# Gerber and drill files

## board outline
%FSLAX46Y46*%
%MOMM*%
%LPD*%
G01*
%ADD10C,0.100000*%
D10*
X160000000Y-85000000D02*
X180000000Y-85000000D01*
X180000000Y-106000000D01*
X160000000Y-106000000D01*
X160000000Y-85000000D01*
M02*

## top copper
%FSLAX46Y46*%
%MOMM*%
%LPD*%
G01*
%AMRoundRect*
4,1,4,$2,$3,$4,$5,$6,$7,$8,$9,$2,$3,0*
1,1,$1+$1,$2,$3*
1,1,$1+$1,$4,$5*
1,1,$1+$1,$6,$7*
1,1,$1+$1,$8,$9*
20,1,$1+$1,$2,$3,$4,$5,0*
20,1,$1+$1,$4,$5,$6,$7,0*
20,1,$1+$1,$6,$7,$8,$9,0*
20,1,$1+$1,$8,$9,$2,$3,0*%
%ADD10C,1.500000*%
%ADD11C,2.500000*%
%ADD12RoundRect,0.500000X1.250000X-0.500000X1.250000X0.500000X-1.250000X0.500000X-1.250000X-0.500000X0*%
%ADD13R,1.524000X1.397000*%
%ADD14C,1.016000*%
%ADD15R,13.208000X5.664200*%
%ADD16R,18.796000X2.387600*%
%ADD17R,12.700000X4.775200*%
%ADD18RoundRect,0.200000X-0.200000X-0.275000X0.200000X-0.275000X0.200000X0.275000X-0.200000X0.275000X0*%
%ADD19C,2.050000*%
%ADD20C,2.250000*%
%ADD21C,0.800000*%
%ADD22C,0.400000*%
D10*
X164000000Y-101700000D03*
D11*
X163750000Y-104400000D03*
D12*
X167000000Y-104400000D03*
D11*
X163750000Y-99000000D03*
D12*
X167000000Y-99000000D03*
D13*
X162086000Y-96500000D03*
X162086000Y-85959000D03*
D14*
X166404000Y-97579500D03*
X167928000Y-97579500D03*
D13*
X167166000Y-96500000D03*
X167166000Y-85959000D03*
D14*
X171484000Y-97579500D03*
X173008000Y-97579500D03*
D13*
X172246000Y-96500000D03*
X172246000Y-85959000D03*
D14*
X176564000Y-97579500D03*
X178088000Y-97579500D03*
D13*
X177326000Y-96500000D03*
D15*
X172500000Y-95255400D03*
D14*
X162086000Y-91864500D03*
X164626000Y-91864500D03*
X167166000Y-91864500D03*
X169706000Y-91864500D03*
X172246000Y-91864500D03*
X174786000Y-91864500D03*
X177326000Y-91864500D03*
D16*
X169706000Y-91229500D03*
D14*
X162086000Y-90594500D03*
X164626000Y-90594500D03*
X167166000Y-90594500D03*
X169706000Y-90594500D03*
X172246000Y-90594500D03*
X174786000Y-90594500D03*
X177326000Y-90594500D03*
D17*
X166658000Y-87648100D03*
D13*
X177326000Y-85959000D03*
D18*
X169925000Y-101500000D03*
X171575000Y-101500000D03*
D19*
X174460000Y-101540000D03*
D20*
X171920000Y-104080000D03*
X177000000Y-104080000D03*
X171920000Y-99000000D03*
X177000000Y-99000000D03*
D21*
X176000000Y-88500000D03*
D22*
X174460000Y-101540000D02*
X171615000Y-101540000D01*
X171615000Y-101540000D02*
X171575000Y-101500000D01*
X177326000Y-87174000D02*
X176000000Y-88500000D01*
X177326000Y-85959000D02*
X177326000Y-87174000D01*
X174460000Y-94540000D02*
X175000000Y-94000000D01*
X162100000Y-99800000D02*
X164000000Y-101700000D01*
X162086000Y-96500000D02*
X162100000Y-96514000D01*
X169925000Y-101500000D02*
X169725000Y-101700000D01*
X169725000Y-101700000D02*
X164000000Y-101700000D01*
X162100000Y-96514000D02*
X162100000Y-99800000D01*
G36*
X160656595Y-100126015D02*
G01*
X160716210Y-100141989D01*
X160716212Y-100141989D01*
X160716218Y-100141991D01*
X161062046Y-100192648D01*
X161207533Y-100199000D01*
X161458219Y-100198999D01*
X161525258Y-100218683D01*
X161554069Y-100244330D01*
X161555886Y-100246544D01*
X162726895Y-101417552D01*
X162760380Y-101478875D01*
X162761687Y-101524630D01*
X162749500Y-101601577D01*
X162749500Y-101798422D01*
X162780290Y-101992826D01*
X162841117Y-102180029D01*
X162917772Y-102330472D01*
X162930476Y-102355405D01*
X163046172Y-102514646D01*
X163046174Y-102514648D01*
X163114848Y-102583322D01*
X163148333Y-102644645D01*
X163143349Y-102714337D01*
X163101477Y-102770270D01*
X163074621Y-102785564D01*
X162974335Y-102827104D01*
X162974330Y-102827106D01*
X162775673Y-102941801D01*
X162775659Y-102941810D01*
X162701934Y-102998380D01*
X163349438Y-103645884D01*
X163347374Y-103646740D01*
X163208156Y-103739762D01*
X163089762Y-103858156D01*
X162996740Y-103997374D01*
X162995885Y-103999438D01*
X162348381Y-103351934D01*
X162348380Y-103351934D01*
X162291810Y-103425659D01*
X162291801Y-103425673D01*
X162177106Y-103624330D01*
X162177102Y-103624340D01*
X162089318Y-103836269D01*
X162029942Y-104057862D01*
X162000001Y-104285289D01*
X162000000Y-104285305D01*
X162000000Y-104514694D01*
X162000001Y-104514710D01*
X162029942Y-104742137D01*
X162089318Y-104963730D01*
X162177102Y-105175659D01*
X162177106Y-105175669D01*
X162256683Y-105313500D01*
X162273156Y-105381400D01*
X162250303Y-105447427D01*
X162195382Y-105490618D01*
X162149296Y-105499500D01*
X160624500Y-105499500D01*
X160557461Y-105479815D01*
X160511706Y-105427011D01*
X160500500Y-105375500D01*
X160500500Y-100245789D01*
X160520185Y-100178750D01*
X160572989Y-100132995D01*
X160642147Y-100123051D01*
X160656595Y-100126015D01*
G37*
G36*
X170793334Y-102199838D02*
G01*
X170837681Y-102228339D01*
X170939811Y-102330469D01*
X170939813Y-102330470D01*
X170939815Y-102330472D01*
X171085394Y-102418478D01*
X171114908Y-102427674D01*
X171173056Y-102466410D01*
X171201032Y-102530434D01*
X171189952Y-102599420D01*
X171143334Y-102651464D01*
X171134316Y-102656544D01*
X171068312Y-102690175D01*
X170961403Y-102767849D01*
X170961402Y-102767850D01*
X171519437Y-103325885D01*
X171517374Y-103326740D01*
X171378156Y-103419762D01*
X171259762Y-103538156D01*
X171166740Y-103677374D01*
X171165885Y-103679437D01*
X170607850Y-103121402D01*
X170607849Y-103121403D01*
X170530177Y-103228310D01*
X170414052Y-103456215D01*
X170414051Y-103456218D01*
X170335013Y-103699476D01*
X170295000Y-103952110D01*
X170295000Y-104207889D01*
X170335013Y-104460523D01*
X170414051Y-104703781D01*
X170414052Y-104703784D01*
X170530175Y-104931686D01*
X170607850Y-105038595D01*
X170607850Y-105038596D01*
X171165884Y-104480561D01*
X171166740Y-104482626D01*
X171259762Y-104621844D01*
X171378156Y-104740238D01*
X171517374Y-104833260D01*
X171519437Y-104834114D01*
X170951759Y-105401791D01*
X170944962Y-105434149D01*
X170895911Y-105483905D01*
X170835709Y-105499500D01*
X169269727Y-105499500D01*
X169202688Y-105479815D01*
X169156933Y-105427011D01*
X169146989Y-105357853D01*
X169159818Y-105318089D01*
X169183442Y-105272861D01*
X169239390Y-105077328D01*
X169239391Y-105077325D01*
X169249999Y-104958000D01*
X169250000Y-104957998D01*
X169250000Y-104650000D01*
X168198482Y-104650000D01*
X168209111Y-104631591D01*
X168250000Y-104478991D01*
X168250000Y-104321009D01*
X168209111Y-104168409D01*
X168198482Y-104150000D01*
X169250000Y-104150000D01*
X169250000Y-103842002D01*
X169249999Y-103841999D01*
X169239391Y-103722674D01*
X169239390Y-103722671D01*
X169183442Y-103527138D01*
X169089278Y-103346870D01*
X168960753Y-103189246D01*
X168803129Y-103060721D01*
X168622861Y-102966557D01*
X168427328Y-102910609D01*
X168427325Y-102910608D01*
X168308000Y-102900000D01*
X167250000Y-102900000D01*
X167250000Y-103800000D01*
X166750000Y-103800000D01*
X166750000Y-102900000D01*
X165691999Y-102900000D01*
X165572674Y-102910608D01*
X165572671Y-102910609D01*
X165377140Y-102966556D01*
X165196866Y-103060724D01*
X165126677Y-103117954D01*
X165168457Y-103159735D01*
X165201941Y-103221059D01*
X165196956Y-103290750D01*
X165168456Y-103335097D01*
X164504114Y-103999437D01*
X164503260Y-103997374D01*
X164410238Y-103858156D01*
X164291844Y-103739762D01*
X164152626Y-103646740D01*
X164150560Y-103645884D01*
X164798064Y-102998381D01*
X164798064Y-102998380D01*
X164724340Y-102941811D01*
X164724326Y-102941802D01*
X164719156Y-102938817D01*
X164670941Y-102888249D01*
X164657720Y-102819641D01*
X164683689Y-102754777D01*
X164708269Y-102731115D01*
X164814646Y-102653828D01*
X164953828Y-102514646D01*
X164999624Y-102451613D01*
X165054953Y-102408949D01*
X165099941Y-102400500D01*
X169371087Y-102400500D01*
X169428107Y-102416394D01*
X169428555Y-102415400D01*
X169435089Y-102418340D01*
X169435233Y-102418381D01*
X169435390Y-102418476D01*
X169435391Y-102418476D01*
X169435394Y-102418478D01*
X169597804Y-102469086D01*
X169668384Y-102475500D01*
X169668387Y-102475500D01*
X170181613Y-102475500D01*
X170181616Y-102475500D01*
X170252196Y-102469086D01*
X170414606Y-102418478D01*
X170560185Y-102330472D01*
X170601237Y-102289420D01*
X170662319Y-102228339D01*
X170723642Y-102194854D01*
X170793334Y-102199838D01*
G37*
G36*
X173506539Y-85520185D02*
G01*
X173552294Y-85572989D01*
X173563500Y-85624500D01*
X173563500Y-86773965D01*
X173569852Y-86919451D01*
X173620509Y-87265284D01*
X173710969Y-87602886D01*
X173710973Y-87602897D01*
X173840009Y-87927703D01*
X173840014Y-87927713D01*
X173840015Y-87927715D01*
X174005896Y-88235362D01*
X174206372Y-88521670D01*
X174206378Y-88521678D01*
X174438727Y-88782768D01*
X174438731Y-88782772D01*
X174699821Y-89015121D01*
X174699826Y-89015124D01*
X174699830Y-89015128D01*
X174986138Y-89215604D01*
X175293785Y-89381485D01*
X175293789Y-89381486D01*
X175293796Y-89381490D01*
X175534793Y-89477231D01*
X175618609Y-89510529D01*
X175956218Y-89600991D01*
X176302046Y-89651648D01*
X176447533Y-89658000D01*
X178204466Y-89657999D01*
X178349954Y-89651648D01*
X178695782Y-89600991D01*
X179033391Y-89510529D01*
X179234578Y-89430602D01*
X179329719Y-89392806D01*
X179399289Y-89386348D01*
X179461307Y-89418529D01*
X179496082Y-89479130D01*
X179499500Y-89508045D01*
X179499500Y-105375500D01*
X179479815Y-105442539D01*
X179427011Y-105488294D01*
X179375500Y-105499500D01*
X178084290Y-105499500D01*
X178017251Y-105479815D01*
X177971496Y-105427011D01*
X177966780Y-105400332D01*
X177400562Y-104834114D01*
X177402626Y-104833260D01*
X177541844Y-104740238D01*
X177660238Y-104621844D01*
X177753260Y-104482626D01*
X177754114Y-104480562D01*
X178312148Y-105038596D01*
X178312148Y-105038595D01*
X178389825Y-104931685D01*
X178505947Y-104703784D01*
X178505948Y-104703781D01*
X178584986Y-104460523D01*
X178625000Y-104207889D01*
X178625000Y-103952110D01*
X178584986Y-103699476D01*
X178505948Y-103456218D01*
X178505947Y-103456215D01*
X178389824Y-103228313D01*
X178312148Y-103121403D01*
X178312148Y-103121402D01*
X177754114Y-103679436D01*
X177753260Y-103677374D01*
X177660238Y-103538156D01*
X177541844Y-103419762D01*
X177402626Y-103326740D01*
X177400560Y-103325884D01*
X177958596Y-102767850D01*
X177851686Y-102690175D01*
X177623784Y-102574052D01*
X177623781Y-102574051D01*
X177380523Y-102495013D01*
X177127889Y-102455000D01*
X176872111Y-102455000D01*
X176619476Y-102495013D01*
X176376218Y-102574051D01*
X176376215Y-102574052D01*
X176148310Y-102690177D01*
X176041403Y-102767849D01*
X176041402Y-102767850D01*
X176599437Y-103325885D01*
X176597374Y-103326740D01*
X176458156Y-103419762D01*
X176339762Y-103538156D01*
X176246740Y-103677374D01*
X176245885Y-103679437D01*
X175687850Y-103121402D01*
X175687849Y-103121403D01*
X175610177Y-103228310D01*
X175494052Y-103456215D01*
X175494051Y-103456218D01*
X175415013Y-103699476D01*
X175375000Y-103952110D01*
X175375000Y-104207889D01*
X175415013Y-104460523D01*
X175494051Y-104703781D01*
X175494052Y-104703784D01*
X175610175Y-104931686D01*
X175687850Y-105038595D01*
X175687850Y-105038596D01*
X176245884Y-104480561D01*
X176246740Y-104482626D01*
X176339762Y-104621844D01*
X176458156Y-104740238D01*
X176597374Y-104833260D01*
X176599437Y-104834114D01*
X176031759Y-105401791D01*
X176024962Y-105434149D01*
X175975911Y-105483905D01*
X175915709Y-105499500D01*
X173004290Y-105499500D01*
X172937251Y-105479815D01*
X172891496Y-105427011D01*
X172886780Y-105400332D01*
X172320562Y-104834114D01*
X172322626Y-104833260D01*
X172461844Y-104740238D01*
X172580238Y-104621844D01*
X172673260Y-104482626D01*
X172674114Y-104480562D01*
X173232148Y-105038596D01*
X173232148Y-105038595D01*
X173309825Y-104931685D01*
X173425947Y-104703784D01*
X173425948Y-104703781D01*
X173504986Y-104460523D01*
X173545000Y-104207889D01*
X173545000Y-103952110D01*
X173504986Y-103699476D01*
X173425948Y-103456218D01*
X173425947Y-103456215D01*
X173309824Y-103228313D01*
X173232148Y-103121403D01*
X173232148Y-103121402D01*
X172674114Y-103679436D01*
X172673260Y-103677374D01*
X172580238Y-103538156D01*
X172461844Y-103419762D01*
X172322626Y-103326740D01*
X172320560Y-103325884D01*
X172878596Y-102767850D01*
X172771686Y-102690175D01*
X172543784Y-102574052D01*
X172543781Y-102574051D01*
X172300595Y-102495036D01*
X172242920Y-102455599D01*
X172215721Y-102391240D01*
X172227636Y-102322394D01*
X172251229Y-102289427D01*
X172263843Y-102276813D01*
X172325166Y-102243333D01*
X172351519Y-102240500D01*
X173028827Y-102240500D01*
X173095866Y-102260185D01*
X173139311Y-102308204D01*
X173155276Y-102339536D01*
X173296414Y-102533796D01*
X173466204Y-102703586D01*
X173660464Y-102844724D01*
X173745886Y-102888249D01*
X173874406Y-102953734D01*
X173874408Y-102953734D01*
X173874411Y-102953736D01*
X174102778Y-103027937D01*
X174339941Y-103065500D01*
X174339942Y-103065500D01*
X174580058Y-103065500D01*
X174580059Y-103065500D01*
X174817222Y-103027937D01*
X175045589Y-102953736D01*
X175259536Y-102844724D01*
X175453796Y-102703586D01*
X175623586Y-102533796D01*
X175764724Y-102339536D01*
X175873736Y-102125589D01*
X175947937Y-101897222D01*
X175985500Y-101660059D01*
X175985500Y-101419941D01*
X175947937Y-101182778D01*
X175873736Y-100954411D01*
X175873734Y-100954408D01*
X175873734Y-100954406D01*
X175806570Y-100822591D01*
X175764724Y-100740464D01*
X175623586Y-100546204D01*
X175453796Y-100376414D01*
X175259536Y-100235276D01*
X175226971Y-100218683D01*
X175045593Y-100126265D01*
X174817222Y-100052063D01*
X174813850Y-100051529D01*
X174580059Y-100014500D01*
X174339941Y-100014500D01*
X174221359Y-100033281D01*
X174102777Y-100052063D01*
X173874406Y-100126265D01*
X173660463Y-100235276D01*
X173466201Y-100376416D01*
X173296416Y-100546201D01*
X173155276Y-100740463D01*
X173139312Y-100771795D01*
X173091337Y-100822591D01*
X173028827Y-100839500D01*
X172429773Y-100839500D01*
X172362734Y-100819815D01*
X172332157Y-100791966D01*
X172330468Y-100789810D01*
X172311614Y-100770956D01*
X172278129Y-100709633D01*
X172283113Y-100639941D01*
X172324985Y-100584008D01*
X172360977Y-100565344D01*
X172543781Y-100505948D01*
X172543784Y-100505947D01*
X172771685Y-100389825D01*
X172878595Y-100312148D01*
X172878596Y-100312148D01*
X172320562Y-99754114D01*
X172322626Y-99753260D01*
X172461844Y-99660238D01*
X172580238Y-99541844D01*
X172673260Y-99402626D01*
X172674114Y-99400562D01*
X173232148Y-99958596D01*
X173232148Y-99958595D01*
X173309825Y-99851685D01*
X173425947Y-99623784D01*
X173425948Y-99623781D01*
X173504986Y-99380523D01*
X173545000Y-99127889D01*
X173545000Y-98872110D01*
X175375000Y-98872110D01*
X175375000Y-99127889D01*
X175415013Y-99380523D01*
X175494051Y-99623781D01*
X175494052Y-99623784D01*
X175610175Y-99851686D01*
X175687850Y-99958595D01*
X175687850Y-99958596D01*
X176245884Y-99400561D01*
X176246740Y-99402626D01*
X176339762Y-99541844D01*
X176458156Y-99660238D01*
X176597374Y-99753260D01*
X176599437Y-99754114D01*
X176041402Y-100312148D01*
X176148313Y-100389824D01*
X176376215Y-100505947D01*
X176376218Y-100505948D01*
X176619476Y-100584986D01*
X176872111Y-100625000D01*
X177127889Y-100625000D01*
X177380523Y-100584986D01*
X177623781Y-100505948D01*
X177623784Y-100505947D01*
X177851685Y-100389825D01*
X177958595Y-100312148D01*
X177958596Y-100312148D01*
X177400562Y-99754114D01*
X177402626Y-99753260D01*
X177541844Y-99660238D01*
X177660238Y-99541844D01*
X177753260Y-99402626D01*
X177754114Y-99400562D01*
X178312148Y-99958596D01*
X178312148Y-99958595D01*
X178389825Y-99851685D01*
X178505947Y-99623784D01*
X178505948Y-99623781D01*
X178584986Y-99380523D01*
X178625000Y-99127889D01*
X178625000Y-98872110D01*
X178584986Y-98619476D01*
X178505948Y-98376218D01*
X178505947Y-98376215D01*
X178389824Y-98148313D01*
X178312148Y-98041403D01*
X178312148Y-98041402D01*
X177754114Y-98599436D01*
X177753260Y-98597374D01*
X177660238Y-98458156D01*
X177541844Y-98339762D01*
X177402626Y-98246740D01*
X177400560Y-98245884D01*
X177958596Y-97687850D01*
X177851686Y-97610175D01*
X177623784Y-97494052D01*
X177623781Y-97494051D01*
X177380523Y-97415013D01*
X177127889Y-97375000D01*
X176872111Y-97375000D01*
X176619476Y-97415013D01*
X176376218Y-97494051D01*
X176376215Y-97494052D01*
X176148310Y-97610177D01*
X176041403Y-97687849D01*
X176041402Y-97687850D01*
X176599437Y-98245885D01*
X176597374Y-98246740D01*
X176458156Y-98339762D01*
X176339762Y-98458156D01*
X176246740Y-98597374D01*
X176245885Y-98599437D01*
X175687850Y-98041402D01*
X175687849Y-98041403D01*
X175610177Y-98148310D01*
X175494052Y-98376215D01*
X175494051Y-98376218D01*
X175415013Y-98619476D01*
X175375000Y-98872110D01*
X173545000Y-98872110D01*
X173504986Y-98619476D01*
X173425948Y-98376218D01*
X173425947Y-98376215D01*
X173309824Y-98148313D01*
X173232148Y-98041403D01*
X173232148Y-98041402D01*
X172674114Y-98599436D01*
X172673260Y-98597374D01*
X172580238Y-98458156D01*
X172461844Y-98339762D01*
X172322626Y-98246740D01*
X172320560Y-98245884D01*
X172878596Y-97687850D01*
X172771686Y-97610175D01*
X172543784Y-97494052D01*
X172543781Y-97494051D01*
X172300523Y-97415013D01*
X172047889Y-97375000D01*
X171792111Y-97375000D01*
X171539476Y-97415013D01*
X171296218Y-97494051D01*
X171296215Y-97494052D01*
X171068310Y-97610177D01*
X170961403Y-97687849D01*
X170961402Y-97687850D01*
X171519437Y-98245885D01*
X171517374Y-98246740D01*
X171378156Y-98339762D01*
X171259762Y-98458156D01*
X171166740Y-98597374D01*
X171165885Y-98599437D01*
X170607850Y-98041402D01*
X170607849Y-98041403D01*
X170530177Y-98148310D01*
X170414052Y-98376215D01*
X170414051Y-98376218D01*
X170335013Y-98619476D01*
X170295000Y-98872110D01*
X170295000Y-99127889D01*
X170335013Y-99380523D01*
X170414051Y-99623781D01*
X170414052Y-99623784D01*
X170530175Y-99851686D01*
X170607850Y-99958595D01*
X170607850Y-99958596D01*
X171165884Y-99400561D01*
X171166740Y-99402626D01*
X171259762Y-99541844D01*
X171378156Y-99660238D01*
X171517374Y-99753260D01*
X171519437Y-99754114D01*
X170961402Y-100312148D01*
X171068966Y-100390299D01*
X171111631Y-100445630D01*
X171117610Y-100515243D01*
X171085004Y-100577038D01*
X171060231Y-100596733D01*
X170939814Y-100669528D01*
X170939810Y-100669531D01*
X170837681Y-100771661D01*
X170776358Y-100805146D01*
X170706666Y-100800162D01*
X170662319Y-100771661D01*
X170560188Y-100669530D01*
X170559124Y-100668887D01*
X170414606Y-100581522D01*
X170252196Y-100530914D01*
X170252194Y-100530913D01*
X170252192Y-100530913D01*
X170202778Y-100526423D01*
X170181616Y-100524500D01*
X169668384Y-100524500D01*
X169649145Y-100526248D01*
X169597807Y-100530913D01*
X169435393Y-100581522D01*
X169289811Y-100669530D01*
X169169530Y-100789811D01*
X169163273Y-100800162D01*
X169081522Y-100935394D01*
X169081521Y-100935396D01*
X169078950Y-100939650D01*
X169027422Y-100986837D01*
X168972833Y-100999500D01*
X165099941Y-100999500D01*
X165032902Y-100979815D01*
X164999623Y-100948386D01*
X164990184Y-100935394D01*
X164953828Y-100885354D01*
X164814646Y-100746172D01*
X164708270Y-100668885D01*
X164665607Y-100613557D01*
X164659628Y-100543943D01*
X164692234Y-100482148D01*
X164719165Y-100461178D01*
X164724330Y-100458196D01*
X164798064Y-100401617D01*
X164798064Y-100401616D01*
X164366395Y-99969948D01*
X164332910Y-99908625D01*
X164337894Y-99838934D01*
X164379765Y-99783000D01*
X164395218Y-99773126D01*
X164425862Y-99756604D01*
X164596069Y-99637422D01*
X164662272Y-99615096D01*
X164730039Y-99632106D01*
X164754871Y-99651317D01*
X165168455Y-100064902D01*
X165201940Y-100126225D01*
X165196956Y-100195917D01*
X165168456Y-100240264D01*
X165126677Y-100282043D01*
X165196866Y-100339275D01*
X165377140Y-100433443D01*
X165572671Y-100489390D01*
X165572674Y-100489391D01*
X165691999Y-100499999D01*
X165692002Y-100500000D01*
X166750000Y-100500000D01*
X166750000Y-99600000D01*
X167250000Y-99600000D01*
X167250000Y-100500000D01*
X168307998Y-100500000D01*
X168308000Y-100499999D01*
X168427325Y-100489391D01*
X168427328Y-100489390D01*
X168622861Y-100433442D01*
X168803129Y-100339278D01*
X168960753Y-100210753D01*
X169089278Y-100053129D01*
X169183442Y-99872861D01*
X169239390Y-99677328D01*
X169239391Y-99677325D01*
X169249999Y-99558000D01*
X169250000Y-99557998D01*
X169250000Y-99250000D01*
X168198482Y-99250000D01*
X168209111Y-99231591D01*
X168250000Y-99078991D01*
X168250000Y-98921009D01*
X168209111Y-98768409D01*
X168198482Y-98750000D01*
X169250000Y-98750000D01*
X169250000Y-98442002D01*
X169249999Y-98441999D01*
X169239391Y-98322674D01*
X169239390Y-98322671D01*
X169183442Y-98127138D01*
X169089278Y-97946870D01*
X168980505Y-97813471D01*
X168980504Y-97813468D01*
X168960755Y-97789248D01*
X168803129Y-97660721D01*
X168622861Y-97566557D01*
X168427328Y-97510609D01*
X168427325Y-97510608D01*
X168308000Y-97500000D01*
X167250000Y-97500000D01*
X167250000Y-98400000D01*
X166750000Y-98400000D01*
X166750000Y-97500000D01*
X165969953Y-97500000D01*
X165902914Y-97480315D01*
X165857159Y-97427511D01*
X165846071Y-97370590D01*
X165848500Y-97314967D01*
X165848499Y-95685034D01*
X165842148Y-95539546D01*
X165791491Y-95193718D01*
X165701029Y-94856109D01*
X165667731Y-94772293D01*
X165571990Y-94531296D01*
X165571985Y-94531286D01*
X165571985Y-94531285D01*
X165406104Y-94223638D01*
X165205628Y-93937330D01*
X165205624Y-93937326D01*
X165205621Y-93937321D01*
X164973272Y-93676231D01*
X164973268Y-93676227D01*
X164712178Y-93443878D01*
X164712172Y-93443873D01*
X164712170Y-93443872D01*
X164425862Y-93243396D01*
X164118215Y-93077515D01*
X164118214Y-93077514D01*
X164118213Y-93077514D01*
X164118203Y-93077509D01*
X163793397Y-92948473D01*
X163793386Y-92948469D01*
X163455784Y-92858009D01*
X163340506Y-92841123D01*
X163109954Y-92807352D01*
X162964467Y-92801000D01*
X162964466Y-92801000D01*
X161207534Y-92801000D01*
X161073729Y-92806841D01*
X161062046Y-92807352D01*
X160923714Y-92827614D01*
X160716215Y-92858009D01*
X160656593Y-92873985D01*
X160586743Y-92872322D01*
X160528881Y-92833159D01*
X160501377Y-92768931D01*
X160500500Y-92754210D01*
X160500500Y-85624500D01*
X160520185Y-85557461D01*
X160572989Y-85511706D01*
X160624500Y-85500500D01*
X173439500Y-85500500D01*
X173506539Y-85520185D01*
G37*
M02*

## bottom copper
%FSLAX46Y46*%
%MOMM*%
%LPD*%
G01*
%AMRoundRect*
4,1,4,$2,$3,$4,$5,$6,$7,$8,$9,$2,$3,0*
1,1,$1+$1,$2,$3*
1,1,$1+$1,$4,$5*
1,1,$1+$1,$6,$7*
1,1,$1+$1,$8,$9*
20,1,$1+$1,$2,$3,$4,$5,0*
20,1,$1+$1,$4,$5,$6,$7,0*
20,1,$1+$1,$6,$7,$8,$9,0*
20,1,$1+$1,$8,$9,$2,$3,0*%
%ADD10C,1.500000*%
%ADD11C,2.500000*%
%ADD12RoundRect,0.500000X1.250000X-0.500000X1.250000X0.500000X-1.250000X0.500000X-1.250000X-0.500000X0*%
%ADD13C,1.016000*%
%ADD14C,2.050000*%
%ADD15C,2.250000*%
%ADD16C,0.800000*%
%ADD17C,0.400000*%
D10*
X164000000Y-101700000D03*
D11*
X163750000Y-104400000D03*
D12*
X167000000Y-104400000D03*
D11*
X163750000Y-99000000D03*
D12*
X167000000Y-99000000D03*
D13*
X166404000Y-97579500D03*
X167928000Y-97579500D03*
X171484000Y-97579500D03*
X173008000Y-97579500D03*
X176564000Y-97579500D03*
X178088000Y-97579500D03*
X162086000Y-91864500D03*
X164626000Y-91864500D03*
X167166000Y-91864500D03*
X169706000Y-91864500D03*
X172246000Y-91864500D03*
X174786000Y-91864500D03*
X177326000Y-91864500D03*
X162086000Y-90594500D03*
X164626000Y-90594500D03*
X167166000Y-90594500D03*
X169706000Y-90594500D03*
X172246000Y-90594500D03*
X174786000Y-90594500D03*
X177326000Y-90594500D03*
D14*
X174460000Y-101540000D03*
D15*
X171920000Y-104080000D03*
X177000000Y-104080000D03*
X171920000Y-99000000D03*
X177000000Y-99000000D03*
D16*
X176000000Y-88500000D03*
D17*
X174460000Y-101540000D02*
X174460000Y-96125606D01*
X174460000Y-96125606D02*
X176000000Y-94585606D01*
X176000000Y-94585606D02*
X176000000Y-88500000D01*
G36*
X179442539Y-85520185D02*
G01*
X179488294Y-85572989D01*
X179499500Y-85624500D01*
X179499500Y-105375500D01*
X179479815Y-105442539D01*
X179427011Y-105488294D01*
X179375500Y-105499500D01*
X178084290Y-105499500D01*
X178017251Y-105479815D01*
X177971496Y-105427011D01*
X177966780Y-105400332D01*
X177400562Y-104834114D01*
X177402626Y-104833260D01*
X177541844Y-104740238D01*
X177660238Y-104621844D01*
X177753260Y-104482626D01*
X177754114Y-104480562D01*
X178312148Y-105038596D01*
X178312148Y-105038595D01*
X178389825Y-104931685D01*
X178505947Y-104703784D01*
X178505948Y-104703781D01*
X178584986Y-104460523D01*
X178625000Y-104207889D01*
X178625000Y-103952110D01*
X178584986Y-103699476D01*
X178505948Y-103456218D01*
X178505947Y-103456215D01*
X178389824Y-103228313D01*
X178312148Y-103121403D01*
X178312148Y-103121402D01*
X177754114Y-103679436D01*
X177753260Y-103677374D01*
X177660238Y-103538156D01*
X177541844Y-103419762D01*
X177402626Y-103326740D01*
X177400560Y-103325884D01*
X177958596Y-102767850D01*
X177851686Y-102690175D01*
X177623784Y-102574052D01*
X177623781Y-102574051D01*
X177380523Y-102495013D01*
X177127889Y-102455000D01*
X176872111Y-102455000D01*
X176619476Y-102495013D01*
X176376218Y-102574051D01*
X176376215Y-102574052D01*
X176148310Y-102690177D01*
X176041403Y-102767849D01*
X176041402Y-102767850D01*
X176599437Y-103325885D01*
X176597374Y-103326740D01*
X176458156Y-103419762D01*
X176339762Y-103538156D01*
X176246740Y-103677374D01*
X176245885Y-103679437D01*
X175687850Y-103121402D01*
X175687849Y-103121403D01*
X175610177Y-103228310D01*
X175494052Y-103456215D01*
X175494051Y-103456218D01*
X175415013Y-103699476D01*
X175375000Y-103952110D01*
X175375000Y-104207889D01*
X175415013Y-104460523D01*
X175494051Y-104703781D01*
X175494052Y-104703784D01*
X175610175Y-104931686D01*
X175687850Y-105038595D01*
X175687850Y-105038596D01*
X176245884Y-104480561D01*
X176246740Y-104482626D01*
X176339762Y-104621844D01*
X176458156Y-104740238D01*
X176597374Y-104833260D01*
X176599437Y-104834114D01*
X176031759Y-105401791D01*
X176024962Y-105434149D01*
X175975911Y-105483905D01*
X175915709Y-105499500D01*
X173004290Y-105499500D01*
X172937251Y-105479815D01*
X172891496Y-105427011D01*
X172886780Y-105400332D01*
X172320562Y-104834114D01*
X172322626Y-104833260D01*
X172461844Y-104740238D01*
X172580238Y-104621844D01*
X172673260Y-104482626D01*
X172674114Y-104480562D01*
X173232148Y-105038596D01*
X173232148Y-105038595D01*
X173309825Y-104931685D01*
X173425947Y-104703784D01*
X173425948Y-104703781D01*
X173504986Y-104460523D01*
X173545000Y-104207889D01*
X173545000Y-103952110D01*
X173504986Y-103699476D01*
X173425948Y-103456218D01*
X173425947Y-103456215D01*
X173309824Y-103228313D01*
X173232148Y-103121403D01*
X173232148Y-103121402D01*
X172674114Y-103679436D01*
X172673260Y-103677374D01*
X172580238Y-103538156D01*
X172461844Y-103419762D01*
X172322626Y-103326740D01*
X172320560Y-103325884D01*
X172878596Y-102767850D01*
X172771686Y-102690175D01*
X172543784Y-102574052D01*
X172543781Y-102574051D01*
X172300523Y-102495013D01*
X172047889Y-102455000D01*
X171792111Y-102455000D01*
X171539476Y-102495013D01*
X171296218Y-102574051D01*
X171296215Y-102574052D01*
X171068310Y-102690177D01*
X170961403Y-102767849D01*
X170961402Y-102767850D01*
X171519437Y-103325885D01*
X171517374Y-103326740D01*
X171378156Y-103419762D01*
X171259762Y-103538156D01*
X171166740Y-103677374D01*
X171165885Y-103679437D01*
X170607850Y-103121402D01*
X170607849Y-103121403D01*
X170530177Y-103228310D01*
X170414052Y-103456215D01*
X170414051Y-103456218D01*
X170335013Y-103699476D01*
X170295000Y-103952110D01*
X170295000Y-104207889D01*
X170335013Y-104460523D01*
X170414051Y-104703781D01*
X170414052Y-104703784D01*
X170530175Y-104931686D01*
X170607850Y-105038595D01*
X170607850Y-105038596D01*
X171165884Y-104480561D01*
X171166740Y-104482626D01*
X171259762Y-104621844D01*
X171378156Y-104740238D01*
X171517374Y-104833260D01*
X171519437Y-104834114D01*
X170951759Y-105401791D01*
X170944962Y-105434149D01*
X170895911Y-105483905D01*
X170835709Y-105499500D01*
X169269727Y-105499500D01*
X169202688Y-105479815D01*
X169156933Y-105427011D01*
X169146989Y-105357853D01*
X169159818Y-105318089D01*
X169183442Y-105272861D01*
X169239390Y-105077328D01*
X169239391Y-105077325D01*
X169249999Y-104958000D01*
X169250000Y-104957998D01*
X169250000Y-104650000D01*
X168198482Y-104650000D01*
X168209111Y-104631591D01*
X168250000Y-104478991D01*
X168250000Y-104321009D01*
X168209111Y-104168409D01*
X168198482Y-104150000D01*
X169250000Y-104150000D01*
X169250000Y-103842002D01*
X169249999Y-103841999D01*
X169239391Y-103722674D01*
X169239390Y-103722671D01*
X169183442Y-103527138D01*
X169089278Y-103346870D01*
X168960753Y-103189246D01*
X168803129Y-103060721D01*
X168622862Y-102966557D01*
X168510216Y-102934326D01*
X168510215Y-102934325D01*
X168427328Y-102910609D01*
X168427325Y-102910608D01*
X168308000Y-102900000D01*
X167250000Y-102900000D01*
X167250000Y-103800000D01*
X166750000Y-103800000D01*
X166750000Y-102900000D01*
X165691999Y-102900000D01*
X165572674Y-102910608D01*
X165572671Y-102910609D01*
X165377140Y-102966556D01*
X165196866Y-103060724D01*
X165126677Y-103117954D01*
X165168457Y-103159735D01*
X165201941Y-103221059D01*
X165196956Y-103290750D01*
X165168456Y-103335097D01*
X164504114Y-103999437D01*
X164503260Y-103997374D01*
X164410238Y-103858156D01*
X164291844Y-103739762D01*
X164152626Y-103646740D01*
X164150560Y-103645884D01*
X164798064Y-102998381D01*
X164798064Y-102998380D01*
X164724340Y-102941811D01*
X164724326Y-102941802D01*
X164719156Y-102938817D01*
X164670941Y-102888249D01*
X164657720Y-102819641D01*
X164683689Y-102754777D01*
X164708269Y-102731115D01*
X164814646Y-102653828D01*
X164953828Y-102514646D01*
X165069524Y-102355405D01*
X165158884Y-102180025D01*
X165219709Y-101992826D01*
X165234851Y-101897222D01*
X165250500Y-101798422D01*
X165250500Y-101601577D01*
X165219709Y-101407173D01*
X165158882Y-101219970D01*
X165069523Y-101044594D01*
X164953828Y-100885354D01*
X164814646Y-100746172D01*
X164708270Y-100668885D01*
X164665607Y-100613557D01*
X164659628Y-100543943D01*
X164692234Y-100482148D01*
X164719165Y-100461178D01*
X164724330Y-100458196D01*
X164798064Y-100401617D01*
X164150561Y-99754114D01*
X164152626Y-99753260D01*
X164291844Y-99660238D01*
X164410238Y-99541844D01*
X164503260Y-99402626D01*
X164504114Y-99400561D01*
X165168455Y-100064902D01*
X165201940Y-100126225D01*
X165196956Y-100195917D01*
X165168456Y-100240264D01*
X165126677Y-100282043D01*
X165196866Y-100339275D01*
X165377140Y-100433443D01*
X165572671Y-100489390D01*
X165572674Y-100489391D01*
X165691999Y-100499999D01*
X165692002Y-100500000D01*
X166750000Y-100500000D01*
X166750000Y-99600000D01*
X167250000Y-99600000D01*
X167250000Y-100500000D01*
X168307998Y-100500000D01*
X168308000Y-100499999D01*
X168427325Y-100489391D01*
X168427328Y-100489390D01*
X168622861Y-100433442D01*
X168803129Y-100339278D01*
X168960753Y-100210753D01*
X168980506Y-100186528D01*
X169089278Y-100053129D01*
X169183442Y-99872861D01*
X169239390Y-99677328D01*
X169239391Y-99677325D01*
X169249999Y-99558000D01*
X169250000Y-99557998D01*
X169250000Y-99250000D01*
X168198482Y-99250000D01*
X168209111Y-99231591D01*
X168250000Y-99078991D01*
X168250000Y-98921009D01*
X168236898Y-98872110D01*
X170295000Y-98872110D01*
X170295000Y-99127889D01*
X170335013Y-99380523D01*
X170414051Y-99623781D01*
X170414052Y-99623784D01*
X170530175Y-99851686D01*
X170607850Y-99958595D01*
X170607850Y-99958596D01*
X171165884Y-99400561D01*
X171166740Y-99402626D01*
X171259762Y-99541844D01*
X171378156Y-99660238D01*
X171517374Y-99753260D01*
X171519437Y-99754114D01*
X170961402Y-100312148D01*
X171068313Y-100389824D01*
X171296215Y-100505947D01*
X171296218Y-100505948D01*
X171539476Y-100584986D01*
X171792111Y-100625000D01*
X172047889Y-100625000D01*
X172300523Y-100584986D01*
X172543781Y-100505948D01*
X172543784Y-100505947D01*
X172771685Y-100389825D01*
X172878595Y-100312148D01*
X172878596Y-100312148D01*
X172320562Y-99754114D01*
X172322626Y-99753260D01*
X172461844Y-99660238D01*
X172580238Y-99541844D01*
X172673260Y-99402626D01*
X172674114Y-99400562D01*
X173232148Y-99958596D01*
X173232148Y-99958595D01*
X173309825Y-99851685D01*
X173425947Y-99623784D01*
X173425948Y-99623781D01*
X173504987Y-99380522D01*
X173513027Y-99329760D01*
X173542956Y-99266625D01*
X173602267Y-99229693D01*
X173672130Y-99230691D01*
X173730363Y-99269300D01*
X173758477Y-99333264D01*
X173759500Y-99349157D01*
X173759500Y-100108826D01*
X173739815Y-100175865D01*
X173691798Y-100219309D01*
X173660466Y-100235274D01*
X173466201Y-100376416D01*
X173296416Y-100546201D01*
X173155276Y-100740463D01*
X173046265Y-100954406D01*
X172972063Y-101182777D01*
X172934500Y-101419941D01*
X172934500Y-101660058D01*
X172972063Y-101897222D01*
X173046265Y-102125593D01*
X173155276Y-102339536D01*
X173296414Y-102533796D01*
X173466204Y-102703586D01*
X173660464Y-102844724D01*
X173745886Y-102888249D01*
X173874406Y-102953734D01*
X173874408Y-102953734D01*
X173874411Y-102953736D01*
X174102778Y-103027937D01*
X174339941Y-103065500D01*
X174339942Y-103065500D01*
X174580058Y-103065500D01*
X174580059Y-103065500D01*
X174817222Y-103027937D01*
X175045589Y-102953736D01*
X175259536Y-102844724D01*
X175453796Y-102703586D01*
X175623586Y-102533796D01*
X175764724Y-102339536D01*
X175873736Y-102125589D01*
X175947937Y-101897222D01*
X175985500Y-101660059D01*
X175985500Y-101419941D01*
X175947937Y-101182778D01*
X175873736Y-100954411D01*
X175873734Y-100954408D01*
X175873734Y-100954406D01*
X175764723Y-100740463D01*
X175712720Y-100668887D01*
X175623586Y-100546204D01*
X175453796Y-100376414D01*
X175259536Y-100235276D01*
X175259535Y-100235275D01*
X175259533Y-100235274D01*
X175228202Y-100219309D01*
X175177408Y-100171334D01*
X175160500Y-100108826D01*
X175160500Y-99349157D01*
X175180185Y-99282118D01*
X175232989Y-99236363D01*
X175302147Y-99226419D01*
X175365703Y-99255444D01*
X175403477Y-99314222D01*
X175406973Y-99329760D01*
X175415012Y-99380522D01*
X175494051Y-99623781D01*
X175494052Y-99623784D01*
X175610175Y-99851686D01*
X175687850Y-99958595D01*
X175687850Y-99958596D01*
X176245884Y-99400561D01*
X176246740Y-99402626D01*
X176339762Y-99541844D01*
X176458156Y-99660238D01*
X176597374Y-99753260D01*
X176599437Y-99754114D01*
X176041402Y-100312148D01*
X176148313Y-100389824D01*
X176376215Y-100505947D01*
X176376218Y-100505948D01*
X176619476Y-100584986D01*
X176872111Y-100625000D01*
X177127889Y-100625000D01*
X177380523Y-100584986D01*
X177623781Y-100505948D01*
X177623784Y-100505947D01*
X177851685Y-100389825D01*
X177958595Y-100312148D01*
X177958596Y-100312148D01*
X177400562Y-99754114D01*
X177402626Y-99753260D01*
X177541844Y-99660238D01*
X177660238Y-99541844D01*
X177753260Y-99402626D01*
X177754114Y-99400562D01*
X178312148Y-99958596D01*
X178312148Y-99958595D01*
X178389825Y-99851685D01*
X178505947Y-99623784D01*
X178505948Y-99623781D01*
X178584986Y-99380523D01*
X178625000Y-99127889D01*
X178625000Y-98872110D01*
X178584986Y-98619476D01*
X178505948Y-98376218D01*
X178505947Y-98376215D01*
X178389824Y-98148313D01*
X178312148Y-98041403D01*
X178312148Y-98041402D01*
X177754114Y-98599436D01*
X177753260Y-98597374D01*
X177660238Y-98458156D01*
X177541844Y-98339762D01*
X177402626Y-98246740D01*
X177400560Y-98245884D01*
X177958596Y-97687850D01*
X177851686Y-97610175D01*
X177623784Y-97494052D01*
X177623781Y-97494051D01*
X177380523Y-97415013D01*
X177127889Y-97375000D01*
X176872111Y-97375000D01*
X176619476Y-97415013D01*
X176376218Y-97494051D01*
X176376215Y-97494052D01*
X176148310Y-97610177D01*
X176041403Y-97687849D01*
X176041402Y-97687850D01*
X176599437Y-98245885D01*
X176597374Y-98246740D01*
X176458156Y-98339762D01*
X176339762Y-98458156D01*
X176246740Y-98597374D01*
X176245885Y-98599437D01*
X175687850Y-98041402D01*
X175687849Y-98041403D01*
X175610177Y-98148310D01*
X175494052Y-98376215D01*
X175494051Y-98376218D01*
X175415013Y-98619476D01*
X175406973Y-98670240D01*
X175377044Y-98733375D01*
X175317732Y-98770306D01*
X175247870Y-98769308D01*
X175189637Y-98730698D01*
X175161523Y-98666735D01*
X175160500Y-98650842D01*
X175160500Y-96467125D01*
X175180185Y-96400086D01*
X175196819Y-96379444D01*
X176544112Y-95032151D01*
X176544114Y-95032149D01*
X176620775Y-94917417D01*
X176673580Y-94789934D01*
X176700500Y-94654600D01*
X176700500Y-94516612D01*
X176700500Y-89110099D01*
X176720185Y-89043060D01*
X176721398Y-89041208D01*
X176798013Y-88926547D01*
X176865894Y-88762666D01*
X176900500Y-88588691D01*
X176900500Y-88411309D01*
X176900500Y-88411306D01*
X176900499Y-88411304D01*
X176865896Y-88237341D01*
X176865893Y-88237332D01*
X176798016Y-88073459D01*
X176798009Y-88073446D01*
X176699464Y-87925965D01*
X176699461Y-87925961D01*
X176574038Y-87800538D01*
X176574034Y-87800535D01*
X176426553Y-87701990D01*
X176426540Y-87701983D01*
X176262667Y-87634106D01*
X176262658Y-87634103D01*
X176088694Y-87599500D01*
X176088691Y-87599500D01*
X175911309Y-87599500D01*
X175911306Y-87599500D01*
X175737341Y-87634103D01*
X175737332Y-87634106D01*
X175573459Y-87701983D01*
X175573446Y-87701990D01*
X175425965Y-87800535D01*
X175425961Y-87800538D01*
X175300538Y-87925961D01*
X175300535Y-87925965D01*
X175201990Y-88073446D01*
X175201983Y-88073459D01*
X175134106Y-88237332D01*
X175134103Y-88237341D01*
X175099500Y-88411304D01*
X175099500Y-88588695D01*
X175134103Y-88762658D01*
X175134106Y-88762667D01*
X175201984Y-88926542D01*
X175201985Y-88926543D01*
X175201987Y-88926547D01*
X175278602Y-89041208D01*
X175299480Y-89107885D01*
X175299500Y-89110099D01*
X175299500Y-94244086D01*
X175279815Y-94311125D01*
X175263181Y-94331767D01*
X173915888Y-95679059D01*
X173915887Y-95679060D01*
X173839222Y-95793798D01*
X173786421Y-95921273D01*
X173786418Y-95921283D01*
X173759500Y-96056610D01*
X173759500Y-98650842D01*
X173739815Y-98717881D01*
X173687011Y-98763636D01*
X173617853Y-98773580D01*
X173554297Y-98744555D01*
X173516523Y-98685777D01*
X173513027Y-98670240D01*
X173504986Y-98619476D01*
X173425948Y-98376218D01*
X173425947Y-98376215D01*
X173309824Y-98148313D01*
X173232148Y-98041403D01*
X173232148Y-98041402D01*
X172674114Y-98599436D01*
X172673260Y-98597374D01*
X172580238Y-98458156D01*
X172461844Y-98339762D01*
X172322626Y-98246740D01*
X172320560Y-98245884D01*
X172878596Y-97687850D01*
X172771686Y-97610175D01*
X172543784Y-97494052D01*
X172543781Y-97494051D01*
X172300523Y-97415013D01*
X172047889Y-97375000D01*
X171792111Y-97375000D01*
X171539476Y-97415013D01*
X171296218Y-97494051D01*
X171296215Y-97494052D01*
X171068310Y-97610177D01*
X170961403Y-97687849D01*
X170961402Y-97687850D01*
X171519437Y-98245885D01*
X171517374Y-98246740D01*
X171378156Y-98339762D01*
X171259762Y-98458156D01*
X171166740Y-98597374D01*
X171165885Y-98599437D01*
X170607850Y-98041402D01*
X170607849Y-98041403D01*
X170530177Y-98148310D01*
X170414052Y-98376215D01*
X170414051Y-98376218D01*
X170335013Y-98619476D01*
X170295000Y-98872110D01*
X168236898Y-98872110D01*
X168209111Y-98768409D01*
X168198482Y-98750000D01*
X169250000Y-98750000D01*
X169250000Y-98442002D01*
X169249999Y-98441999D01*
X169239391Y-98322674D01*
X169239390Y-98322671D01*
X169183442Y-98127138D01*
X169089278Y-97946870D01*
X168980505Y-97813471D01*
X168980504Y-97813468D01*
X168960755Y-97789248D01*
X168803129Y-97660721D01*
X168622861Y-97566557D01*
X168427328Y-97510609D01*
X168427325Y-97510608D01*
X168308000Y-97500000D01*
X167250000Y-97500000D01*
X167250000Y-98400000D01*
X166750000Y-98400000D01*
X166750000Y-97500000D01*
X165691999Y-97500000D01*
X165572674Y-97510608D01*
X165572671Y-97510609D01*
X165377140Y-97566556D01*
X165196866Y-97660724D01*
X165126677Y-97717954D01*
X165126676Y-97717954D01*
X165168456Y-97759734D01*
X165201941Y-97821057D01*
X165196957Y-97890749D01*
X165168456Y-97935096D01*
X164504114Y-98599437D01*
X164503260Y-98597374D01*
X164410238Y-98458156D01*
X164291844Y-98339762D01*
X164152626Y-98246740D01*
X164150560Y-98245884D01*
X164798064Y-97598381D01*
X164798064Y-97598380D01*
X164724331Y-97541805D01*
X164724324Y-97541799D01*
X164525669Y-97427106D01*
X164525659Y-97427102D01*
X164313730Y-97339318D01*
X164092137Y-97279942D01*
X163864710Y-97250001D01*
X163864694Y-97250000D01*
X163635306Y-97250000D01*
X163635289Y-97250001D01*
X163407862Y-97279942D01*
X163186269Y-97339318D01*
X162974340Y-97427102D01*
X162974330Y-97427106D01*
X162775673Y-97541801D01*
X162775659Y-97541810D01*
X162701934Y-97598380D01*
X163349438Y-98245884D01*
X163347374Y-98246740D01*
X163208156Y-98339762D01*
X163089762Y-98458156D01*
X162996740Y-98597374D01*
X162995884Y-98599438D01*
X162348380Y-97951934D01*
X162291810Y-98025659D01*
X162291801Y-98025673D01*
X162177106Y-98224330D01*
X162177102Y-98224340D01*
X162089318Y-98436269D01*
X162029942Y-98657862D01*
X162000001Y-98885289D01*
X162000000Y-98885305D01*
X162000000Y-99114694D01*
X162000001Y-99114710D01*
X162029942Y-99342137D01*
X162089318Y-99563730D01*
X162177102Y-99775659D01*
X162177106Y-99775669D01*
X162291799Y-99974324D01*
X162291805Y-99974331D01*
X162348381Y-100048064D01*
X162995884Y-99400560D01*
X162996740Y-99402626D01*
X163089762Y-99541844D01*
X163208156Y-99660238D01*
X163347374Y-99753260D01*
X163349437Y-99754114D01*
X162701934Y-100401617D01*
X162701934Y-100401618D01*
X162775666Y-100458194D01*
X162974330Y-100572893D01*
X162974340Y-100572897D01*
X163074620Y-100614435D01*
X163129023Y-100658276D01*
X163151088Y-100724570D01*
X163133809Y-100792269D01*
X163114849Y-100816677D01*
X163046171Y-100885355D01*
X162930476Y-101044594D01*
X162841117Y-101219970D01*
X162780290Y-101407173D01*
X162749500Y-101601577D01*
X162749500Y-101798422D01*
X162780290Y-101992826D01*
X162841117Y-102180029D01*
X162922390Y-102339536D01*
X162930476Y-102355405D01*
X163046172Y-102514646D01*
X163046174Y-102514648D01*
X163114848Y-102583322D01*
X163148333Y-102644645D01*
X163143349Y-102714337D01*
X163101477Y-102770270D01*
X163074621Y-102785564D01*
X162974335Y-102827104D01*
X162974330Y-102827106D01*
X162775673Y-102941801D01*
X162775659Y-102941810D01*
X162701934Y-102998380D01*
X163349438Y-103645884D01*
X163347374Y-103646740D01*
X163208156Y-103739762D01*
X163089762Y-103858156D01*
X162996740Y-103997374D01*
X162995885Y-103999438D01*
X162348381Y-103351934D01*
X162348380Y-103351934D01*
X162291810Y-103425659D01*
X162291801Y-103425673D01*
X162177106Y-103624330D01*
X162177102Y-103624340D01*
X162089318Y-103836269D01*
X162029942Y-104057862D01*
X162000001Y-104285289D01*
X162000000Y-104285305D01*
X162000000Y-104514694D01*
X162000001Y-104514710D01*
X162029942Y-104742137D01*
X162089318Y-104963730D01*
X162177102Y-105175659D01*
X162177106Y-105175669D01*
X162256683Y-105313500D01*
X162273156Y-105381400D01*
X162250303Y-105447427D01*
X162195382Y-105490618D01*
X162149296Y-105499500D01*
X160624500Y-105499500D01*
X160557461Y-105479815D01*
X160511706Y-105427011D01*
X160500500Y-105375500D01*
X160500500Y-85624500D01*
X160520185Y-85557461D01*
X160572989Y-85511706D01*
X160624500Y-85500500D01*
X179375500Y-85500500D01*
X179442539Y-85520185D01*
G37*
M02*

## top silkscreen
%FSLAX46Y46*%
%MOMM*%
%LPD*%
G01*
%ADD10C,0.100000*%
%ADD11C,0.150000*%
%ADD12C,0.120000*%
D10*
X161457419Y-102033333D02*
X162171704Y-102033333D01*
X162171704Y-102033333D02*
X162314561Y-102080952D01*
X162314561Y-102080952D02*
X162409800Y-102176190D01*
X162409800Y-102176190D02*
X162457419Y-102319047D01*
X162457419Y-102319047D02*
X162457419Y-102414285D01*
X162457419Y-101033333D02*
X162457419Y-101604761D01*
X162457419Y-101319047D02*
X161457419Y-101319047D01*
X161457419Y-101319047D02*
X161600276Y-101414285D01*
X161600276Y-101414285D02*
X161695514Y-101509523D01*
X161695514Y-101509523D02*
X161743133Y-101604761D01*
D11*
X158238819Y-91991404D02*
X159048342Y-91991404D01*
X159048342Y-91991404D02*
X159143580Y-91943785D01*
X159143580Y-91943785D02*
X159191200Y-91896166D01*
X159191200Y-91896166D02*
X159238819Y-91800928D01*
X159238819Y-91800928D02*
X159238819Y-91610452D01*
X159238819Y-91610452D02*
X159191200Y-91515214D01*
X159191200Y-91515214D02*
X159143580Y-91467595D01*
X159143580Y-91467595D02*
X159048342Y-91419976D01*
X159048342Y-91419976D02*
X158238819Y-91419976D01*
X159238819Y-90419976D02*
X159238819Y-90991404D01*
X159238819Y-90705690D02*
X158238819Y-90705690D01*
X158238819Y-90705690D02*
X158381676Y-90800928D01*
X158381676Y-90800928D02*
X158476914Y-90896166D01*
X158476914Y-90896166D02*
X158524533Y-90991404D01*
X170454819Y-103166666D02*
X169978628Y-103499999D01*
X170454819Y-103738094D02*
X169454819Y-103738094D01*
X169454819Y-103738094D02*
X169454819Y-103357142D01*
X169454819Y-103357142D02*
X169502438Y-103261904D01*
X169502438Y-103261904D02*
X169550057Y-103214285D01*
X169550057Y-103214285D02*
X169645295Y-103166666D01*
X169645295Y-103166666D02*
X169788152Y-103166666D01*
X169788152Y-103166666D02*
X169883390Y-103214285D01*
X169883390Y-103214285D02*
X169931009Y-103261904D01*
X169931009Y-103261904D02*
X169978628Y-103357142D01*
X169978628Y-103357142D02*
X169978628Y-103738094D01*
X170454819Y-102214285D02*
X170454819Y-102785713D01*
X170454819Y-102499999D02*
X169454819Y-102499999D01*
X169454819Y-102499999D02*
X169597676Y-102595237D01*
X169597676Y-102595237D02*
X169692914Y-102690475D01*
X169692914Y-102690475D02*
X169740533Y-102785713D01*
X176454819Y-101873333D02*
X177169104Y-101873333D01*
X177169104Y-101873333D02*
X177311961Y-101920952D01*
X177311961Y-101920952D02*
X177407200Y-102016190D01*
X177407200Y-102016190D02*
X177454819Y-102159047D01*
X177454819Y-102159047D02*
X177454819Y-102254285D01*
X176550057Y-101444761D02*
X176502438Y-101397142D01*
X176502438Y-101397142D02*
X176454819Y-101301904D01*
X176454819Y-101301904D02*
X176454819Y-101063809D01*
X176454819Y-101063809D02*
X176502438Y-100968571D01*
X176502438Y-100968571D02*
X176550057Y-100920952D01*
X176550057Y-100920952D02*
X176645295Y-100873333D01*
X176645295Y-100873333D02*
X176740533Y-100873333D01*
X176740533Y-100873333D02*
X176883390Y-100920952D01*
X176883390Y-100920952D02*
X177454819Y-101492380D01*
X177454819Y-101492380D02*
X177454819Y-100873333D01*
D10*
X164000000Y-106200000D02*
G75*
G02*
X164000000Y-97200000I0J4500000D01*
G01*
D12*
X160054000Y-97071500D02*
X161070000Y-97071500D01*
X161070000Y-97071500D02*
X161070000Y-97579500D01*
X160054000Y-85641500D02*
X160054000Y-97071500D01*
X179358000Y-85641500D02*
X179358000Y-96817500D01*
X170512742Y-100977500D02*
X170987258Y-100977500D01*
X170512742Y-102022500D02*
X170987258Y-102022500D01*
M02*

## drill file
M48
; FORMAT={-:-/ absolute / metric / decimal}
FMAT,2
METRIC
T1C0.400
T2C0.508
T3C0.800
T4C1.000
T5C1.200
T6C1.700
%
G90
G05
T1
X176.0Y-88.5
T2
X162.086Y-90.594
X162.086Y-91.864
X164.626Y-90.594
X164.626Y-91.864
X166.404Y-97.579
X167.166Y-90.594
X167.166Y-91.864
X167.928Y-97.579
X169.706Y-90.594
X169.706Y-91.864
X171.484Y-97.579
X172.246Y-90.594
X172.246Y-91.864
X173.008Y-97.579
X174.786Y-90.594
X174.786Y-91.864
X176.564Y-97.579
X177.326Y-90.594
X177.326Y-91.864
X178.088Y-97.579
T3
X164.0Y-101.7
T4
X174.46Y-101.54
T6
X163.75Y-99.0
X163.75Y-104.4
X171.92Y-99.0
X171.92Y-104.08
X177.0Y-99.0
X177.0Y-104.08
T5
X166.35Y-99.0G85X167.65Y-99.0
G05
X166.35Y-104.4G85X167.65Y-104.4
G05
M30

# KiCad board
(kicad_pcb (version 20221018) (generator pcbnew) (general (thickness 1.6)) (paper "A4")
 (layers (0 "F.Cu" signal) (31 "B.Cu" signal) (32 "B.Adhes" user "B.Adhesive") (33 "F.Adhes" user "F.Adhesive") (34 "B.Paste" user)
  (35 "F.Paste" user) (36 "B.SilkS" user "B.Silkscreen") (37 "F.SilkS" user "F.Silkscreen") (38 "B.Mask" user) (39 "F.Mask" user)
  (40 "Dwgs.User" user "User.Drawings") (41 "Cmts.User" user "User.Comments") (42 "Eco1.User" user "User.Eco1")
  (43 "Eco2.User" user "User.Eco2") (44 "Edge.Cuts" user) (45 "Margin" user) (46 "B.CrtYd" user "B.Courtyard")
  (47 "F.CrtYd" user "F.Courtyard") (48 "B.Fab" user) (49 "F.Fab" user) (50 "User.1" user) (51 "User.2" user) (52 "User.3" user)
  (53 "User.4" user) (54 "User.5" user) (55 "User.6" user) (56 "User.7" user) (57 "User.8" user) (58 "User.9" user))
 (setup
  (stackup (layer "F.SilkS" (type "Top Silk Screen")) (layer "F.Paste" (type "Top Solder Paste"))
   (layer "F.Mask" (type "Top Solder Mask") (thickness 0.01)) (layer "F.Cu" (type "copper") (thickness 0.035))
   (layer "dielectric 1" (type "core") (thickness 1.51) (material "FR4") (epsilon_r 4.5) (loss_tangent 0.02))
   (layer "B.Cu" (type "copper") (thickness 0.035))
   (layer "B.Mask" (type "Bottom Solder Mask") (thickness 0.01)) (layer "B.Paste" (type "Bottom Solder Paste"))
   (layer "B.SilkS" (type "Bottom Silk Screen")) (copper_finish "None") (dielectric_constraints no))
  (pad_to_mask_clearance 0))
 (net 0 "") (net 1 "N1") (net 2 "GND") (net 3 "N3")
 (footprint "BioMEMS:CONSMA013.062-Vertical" (layer "F.Cu") (at 164 101.7 90)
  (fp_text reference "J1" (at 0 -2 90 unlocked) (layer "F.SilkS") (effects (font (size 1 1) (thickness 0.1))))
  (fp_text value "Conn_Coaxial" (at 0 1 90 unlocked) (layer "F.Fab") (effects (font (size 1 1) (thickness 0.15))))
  (fp_arc (start -4.5 0) (mid 0 -4.5) (end 4.5 0) (stroke (width 0.1) (type default)) (layer "F.SilkS"))
  (pad "1" thru_hole circle (at 0 0 90) (size 1.5 1.5) (drill 0.8) (layers "*.Cu" "*.Mask") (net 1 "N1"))
  (pad "2" thru_hole circle (at -2.7 -0.25 90) (size 2.5 2.5) (drill 1.7) (layers "*.Cu" "*.Mask") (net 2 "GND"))
  (pad "2" thru_hole roundrect (at -2.7 3 90) (size 2 3.5) (drill oval 1.2 2.5) (layers "*.Cu" "*.Mask") (roundrect_rratio 0.25)
   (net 2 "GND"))
  (pad "2" thru_hole circle (at 2.7 -0.25 90) (size 2.5 2.5) (drill 1.7) (layers "*.Cu" "*.Mask") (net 2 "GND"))
  (pad "2" thru_hole roundrect (at 2.7 3 90) (size 2 3.5) (drill oval 1.2 2.5) (layers "*.Cu" "*.Mask") (roundrect_rratio 0.25)
   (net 2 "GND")))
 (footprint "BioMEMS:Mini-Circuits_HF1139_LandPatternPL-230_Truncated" (layer "F.Cu") (at 169.706 91.2295 90)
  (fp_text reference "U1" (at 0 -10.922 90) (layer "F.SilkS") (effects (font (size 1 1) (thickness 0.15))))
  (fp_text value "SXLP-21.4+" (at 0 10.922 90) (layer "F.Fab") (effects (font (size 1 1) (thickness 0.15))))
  (fp_line (start -5.842 -9.652) (end -5.842 -8.636) (stroke (width 0.12) (type solid)) (layer "F.SilkS"))
  (fp_line (start -5.842 -8.636) (end -6.35 -8.636) (stroke (width 0.12) (type solid)) (layer "F.SilkS"))
  (fp_line (start 5.588 -9.652) (end -5.842 -9.652) (stroke (width 0.12) (type solid)) (layer "F.SilkS"))
  (fp_line (start 5.588 9.652) (end -5.588 9.652) (stroke (width 0.12) (type solid)) (layer "F.SilkS"))
  (pad "1" smd rect (at -5.2705 -7.62) (size 1.524 1.397) (layers "F.Cu" "F.Paste" "F.Mask") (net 1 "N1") (clearance 3))
  (pad "2" smd rect (at 5.2705 -7.62) (size 1.524 1.397) (layers "F.Cu" "F.Paste" "F.Mask") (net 2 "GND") (zone_connect 2))
  (pad "3" thru_hole circle (at -6.35 -3.302) (size 1.016 1.016) (drill 0.508) (layers "*.Cu") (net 2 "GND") (zone_connect 2))
  (pad "3" thru_hole circle (at -6.35 -1.778) (size 1.016 1.016) (drill 0.508) (layers "*.Cu") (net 2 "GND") (zone_connect 2))
  (pad "3" smd rect (at -5.2705 -2.54) (size 1.524 1.397) (layers "F.Cu" "F.Paste" "F.Mask") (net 2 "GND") (zone_connect 2))
  (pad "4" smd rect (at 5.2705 -2.54) (size 1.524 1.397) (layers "F.Cu" "F.Paste" "F.Mask") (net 2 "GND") (zone_connect 2))
  (pad "5" thru_hole circle (at -6.35 1.778) (size 1.016 1.016) (drill 0.508) (layers "*.Cu") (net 2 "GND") (zone_connect 2))
  (pad "5" thru_hole circle (at -6.35 3.302) (size 1.016 1.016) (drill 0.508) (layers "*.Cu") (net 2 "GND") (zone_connect 2))
  (pad "5" smd rect (at -5.2705 2.54) (size 1.524 1.397) (layers "F.Cu" "F.Paste" "F.Mask") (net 2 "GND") (zone_connect 2))
  (pad "6" smd rect (at 5.2705 2.54) (size 1.524 1.397) (layers "F.Cu" "F.Paste" "F.Mask") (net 2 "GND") (zone_connect 2))
  (pad "7" thru_hole circle (at -6.35 6.858) (size 1.016 1.016) (drill 0.508) (layers "*.Cu") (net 2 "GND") (zone_connect 2))
  (pad "7" thru_hole circle (at -6.35 8.382) (size 1.016 1.016) (drill 0.508) (layers "*.Cu") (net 2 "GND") (zone_connect 2))
  (pad "7" smd rect (at -5.2705 7.62) (size 1.524 1.397) (layers "F.Cu" "F.Paste" "F.Mask") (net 2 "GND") (zone_connect 2))
  (pad "7" smd rect (at -4.0259 2.794) (size 13.208 5.6642) (layers "F.Cu") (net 2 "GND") (zone_connect 2))
  (pad "7" thru_hole circle (at -0.635 -7.62) (size 1.016 1.016) (drill 0.508) (layers "*.Cu") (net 2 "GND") (zone_connect 2))
  (pad "7" thru_hole circle (at -0.635 -5.08) (size 1.016 1.016) (drill 0.508) (layers "*.Cu") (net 2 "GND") (zone_connect 2))
  (pad "7" thru_hole circle (at -0.635 -2.54) (size 1.016 1.016) (drill 0.508) (layers "*.Cu") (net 2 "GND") (zone_connect 2))
  (pad "7" thru_hole circle (at -0.635 0) (size 1.016 1.016) (drill 0.508) (layers "*.Cu") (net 2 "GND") (zone_connect 2))
  (pad "7" thru_hole circle (at -0.635 2.54) (size 1.016 1.016) (drill 0.508) (layers "*.Cu") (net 2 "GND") (zone_connect 2))
  (pad "7" thru_hole circle (at -0.635 5.08) (size 1.016 1.016) (drill 0.508) (layers "*.Cu") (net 2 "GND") (zone_connect 2))
  (pad "7" thru_hole circle (at -0.635 7.62) (size 1.016 1.016) (drill 0.508) (layers "*.Cu") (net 2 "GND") (zone_connect 2))
  (pad "7" smd rect (at 0 0) (size 18.796 2.3876) (layers "F.Cu") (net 2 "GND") (zone_connect 2))
  (pad "7" thru_hole circle (at 0.635 -7.62) (size 1.016 1.016) (drill 0.508) (layers "*.Cu") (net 2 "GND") (zone_connect 2))
  (pad "7" thru_hole circle (at 0.635 -5.08) (size 1.016 1.016) (drill 0.508) (layers "*.Cu") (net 2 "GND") (zone_connect 2))
  (pad "7" thru_hole circle (at 0.635 -2.54) (size 1.016 1.016) (drill 0.508) (layers "*.Cu") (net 2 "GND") (zone_connect 2))
  (pad "7" thru_hole circle (at 0.635 0) (size 1.016 1.016) (drill 0.508) (layers "*.Cu") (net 2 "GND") (zone_connect 2))
  (pad "7" thru_hole circle (at 0.635 2.54) (size 1.016 1.016) (drill 0.508) (layers "*.Cu") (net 2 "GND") (zone_connect 2))
  (pad "7" thru_hole circle (at 0.635 5.08) (size 1.016 1.016) (drill 0.508) (layers "*.Cu") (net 2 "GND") (zone_connect 2))
  (pad "7" thru_hole circle (at 0.635 7.62) (size 1.016 1.016) (drill 0.508) (layers "*.Cu") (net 2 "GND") (zone_connect 2))
  (pad "7" smd rect (at 3.5814 -3.048) (size 12.7 4.7752) (layers "F.Cu") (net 2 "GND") (zone_connect 2))
  (pad "8" smd rect (at 5.2705 7.62) (size 1.524 1.397) (layers "F.Cu" "F.Paste" "F.Mask") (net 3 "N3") (clearance 3)))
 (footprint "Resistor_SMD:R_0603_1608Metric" (layer "F.Cu") (at 170.75 101.5)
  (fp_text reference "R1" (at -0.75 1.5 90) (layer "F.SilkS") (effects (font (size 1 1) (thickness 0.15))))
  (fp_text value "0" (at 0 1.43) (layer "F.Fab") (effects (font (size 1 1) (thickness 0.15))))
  (fp_line (start -0.237258 -0.5225) (end 0.237258 -0.5225) (stroke (width 0.12) (type solid)) (layer "F.SilkS"))
  (fp_line (start -0.237258 0.5225) (end 0.237258 0.5225) (stroke (width 0.12) (type solid)) (layer "F.SilkS"))
  (pad "1" smd roundrect (at -0.825 0) (size 0.8 0.95) (layers "F.Cu" "F.Paste" "F.Mask") (roundrect_rratio 0.25) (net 1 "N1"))
  (pad "2" smd roundrect (at 0.825 0) (size 0.8 0.95) (layers "F.Cu" "F.Paste" "F.Mask") (roundrect_rratio 0.25) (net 3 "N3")))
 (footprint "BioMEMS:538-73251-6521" (layer "B.Cu") (at 174.46 101.54 90)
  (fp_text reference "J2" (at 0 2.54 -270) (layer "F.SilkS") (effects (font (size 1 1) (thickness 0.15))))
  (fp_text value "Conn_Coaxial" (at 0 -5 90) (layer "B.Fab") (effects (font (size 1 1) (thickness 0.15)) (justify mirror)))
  (pad "1" thru_hole circle (at 0 0 90) (size 2.05 2.05) (drill 1) (layers "*.Cu" "*.Mask") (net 3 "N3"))
  (pad "2" thru_hole circle (at -2.54 -2.54 90) (size 2.25 2.25) (drill 1.7) (layers "*.Cu" "*.Mask") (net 2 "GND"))
  (pad "2" thru_hole circle (at -2.54 2.54 90) (size 2.25 2.25) (drill 1.7) (layers "*.Cu" "*.Mask") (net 2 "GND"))
  (pad "2" thru_hole circle (at 2.54 -2.54 90) (size 2.25 2.25) (drill 1.7) (layers "*.Cu" "*.Mask") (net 2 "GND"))
  (pad "2" thru_hole circle (at 2.54 2.54 90) (size 2.25 2.25) (drill 1.7) (layers "*.Cu" "*.Mask") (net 2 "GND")))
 (gr_rect (start 160 85) (end 180 106) (stroke (width 0.1) (type default)) (fill none) (layer "Edge.Cuts"))
 (segment (start 174.46 101.54) (end 171.615 101.54) (width 0.4) (layer "F.Cu") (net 3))
 (segment (start 171.615 101.54) (end 171.575 101.5) (width 0.4) (layer "F.Cu") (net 3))
 (segment (start 177.326 87.174) (end 176 88.5) (width 0.4) (layer "F.Cu") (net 3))
 (segment (start 177.326 85.959) (end 177.326 87.174) (width 0.4) (layer "F.Cu") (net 3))
 (via (at 176 88.5) (size 0.8) (drill 0.4) (layers "F.Cu" "B.Cu") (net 3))
 (segment (start 174.46 101.54) (end 174.46 96.125606) (width 0.4) (layer "B.Cu") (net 3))
 (segment (start 174.46 96.125606) (end 176 94.585606) (width 0.4) (layer "B.Cu") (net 3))
 (segment (start 176 94.585606) (end 176 88.5) (width 0.4) (layer "B.Cu") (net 3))
 (segment (start 174.46 94.54) (end 175 94) (width 0.4) (layer "F.Cu") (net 2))
 (segment (start 162.1 99.8) (end 164 101.7) (width 0.4) (layer "F.Cu") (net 1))
 (segment (start 162.086 96.5) (end 162.1 96.514) (width 0.4) (layer "F.Cu") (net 1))
 (segment (start 169.925 101.5) (end 169.725 101.7) (width 0.4) (layer "F.Cu") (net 1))
 (segment (start 169.725 101.7) (end 164 101.7) (width 0.4) (layer "F.Cu") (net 1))
 (segment (start 162.1 96.514) (end 162.1 99.8) (width 0.4) (layer "F.Cu") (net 1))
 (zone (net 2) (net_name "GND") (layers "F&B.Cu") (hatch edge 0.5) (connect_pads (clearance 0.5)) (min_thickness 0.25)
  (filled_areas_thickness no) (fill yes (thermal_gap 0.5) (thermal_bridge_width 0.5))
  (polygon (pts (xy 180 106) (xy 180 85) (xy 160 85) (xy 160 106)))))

